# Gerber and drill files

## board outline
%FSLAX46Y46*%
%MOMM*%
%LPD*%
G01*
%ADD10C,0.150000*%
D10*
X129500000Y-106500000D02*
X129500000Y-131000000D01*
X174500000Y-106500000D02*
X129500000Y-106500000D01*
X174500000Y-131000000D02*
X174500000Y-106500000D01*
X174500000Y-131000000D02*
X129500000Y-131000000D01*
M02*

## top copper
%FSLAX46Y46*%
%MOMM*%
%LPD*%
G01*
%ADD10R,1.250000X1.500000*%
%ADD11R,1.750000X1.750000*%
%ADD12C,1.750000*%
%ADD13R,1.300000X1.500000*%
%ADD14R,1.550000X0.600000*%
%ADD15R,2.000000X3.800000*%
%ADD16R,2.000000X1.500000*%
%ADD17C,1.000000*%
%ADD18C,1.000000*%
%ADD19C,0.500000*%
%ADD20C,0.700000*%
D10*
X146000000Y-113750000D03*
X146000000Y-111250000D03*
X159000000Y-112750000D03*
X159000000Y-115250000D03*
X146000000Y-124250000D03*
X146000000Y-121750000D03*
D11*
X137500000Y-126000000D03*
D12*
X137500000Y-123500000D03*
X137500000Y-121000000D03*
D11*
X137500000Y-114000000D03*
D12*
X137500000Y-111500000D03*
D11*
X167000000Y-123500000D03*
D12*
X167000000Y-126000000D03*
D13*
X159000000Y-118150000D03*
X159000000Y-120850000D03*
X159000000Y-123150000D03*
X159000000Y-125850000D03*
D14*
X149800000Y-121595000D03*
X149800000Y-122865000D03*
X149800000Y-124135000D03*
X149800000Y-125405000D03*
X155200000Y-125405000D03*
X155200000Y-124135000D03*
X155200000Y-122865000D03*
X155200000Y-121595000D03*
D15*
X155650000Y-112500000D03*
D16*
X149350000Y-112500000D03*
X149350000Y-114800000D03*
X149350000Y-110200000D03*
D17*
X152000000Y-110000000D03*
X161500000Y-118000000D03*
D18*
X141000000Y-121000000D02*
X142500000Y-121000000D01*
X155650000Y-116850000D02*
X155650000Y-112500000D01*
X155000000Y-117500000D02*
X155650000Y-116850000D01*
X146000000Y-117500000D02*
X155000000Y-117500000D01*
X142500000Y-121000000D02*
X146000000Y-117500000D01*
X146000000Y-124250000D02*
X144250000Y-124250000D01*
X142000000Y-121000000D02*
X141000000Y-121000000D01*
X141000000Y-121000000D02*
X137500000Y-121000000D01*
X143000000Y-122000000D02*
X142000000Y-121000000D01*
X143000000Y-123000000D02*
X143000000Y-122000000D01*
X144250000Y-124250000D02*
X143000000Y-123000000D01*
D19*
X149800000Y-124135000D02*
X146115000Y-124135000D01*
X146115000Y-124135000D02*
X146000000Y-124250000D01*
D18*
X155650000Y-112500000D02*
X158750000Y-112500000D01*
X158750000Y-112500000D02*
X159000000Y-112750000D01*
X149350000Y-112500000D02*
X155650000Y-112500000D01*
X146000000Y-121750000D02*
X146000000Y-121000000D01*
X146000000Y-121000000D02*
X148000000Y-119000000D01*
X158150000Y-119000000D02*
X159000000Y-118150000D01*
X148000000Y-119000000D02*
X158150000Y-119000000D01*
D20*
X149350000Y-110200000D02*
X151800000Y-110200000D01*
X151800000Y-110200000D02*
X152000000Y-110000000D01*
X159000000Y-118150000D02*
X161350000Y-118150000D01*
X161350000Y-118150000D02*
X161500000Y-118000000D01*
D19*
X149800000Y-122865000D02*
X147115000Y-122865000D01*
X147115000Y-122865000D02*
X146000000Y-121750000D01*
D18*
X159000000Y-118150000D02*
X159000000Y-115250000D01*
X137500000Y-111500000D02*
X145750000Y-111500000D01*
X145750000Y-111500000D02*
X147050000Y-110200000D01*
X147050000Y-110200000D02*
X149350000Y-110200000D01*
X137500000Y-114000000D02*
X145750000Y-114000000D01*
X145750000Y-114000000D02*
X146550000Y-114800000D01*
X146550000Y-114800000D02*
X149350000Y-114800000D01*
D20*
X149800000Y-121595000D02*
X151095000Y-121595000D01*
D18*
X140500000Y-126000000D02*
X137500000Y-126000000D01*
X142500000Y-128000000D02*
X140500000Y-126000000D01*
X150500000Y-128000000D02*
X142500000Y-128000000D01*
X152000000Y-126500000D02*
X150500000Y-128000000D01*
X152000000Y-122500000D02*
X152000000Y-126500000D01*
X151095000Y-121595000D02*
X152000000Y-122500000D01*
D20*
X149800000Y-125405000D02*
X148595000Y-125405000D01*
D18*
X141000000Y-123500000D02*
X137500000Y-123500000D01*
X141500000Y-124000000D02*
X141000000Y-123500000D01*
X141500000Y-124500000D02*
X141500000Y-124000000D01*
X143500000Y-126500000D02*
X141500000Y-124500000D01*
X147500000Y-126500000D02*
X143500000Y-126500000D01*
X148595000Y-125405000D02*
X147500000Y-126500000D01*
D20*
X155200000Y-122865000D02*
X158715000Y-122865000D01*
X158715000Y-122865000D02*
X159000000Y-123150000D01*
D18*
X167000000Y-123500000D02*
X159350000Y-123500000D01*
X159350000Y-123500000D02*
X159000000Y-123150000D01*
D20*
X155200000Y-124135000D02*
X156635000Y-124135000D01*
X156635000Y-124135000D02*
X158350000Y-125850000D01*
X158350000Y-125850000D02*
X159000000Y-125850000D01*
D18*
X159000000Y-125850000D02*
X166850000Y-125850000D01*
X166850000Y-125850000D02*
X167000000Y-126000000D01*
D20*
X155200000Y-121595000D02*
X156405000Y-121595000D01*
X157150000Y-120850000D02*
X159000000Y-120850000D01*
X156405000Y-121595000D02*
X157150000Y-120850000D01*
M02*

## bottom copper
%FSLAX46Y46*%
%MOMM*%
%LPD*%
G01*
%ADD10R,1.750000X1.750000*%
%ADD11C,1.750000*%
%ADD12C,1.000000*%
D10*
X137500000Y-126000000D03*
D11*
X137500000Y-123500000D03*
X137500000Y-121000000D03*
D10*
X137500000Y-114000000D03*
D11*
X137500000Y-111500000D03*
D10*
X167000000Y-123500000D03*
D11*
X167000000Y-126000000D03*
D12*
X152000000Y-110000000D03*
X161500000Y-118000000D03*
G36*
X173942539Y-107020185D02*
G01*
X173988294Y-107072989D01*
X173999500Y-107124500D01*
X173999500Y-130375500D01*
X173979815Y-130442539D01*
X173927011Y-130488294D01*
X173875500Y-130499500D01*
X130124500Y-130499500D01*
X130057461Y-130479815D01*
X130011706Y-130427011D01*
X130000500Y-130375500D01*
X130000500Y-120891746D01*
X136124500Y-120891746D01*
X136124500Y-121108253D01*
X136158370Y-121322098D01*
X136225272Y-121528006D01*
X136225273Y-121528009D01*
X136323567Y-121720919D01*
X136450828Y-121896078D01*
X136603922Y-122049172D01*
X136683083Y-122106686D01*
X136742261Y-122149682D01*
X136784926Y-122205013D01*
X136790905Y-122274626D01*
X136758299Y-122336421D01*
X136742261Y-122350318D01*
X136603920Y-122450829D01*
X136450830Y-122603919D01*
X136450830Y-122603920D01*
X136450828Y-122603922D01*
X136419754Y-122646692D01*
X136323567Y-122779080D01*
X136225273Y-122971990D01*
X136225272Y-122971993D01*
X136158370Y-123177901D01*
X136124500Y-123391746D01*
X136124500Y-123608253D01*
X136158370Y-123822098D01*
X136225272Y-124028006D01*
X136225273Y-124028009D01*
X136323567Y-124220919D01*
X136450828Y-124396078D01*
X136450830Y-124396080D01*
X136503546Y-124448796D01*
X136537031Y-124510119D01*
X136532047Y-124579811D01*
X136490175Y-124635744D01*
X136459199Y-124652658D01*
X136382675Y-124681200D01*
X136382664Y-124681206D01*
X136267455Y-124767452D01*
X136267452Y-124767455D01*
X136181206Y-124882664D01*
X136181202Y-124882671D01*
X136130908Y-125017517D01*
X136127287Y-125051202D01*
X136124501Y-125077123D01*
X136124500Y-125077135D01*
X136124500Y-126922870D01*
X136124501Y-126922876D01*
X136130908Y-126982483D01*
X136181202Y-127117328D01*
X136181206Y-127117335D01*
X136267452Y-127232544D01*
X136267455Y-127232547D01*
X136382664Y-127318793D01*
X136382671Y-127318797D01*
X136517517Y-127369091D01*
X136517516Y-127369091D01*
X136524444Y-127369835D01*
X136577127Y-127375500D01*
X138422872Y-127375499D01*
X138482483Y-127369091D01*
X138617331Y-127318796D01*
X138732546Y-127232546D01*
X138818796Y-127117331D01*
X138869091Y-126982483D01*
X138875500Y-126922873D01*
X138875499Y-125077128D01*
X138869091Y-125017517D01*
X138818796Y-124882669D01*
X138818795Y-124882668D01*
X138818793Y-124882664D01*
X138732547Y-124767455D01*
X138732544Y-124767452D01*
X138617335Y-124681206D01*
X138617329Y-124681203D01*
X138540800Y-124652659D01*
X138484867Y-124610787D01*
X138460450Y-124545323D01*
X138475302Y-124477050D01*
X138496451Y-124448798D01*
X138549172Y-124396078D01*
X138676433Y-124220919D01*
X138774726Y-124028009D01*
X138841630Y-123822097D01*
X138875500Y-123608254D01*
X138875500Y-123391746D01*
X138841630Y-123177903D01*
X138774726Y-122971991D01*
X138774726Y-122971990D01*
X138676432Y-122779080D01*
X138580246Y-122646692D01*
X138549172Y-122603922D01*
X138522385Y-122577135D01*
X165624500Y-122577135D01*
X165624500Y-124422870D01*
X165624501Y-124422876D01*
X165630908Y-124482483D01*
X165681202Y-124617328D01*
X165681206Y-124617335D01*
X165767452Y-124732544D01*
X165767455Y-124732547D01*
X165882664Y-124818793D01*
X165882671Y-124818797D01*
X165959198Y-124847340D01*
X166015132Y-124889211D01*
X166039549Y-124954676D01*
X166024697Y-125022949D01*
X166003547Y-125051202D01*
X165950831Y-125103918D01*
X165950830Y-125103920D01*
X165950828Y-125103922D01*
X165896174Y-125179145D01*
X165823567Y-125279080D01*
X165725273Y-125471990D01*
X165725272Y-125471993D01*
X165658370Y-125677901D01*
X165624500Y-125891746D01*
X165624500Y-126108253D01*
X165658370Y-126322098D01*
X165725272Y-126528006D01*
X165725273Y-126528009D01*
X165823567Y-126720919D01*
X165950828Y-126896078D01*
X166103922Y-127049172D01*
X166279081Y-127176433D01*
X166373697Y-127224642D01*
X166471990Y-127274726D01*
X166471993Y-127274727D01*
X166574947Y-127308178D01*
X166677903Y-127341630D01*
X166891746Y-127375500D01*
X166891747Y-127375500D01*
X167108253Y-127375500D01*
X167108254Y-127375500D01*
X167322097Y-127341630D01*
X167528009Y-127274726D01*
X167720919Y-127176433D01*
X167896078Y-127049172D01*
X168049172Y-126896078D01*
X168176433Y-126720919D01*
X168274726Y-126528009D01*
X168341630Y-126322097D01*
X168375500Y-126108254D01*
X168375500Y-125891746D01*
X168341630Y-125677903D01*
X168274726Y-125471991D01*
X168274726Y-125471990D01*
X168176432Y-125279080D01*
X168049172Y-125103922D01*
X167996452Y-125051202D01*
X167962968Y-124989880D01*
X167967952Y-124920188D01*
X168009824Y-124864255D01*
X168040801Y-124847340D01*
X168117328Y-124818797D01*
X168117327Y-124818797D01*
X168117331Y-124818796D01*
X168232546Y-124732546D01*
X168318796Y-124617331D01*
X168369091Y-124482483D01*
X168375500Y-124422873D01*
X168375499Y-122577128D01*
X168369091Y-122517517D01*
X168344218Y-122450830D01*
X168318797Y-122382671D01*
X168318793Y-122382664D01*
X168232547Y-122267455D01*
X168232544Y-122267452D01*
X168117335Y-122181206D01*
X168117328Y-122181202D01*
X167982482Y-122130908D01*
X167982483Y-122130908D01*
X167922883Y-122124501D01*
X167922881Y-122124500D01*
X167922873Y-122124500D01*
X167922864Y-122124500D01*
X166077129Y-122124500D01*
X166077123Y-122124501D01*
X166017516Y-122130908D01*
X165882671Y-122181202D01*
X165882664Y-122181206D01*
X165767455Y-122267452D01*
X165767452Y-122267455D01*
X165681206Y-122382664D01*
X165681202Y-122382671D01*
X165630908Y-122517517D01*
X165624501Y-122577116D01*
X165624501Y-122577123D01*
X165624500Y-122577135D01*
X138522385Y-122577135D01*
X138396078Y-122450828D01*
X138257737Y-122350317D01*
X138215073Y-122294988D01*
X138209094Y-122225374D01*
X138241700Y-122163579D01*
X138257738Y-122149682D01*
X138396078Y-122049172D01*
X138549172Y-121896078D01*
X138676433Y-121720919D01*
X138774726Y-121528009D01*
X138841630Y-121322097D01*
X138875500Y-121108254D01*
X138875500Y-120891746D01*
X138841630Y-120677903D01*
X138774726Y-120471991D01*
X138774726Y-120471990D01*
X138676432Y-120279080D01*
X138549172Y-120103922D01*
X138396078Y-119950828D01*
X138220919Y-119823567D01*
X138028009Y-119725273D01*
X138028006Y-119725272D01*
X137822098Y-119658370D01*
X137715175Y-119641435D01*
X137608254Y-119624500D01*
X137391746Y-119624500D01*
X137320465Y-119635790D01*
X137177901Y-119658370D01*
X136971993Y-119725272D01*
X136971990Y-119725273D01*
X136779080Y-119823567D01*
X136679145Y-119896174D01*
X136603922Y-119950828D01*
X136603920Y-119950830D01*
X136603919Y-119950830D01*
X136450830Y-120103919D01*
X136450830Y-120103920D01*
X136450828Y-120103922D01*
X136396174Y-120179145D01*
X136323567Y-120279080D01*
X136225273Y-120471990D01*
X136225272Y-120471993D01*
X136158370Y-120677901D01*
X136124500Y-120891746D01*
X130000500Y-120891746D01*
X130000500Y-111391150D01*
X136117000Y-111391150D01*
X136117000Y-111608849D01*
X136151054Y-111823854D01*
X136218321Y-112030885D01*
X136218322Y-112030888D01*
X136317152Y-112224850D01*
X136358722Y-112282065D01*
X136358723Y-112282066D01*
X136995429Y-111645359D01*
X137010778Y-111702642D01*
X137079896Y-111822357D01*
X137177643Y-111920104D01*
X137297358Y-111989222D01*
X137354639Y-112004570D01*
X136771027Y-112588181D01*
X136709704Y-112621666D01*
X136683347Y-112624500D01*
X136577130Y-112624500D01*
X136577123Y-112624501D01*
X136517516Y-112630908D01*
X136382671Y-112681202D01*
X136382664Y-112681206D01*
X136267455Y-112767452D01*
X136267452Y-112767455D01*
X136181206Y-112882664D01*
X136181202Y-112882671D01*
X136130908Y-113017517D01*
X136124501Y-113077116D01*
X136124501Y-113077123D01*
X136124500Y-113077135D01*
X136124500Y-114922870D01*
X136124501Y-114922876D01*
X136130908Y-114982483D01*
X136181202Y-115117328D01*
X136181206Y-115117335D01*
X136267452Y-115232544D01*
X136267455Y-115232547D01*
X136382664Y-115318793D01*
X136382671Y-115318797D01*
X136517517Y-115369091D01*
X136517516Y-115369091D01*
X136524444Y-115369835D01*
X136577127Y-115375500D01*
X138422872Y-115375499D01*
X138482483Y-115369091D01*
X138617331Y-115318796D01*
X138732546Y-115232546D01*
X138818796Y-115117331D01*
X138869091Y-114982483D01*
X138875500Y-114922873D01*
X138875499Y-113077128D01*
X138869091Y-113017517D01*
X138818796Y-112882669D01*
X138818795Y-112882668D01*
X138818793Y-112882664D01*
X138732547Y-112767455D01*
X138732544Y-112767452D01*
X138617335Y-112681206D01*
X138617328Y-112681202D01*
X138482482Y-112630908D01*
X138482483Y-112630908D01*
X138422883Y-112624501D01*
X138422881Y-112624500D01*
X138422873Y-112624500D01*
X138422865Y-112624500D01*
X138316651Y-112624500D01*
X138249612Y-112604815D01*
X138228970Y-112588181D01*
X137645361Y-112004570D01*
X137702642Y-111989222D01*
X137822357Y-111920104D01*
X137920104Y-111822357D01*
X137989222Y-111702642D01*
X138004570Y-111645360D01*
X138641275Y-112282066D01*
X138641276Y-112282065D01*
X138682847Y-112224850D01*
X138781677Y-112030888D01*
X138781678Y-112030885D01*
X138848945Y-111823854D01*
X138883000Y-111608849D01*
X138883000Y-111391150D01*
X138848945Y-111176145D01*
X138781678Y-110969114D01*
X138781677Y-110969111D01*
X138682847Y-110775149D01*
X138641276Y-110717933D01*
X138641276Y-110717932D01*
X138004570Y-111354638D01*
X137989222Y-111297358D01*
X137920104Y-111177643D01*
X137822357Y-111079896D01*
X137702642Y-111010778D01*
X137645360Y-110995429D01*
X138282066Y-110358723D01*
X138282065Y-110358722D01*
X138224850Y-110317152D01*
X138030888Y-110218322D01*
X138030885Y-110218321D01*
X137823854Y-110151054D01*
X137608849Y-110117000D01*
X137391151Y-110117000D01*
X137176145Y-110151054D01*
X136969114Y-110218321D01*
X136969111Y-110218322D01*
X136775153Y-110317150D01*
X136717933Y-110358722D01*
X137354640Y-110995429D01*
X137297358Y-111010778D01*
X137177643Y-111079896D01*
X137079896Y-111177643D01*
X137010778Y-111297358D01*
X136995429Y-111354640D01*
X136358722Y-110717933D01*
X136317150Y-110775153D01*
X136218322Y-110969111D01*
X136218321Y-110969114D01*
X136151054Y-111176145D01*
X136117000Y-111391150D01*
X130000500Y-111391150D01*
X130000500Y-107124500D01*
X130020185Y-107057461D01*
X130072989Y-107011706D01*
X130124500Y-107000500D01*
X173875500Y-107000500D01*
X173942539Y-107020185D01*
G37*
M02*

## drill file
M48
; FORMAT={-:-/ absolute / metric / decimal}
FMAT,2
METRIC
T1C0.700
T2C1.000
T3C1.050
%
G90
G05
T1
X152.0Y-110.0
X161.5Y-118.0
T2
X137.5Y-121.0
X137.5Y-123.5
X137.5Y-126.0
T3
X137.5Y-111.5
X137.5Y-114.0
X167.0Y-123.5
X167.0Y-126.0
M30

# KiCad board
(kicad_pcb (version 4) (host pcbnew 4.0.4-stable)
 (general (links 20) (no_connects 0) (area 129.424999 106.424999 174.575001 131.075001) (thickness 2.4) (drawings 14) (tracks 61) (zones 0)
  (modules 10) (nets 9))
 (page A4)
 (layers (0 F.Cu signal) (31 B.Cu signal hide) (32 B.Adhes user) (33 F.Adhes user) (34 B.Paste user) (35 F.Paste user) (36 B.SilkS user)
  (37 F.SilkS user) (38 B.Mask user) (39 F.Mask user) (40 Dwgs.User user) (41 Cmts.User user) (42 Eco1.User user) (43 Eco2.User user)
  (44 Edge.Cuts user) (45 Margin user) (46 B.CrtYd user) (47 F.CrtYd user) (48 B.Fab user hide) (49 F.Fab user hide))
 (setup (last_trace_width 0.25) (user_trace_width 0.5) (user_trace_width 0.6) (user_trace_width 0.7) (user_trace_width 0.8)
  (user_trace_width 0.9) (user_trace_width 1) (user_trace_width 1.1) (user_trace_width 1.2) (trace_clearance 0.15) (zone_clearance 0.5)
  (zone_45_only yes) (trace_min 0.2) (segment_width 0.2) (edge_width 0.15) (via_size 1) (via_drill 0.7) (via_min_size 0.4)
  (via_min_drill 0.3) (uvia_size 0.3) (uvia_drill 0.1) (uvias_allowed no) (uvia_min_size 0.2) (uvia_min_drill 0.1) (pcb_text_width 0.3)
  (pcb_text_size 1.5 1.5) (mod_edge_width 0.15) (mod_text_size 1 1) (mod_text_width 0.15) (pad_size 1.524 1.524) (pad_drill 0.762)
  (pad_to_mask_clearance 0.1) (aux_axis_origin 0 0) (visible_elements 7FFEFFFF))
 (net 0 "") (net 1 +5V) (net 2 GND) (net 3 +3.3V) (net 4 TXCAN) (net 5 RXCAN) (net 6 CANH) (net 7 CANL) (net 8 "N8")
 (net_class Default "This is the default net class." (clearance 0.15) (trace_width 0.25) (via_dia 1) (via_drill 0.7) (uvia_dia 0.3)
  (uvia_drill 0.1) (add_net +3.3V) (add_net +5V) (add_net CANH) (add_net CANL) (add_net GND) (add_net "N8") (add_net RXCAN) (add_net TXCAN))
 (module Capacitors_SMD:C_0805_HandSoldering (layer F.Cu) (at 146 112.5 90)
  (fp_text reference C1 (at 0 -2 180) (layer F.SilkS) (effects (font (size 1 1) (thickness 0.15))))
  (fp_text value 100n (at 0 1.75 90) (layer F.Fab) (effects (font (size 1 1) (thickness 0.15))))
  (pad 1 smd rect (at -1.25 0 90) (size 1.5 1.25) (layers F.Cu F.Paste F.Mask) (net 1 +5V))
  (pad 2 smd rect (at 1.25 0 90) (size 1.5 1.25) (layers F.Cu F.Paste F.Mask) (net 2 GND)))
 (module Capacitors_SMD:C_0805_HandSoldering (layer F.Cu) (at 159 114 270)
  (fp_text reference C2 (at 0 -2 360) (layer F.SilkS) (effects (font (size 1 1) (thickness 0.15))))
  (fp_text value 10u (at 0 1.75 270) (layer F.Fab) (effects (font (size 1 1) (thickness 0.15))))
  (pad 1 smd rect (at -1.25 0 270) (size 1.5 1.25) (layers F.Cu F.Paste F.Mask) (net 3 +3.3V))
  (pad 2 smd rect (at 1.25 0 270) (size 1.5 1.25) (layers F.Cu F.Paste F.Mask) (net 2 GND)))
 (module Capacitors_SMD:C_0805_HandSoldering (layer F.Cu) (at 146 123 90)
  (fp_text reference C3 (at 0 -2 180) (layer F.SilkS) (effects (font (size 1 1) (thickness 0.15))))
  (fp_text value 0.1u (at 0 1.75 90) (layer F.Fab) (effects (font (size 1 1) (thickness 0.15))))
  (pad 1 smd rect (at -1.25 0 90) (size 1.5 1.25) (layers F.Cu F.Paste F.Mask) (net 3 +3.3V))
  (pad 2 smd rect (at 1.25 0 90) (size 1.5 1.25) (layers F.Cu F.Paste F.Mask) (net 2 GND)))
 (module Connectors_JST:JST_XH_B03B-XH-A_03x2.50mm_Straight (layer F.Cu) (at 137.5 126 90)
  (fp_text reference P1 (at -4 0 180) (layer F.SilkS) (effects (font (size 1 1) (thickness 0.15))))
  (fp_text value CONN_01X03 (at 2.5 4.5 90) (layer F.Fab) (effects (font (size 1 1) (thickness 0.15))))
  (pad 1 thru_hole rect (at 0 0 90) (size 1.75 1.75) (drill 1) (layers *.Cu *.Mask) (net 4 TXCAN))
  (pad 2 thru_hole circle (at 2.5 0 90) (size 1.75 1.75) (drill 1) (layers *.Cu *.Mask) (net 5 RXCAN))
  (pad 3 thru_hole circle (at 5 0 90) (size 1.75 1.75) (drill 1) (layers *.Cu *.Mask) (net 3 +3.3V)))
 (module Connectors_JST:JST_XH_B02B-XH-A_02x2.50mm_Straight (layer F.Cu) (at 137.5 114 90)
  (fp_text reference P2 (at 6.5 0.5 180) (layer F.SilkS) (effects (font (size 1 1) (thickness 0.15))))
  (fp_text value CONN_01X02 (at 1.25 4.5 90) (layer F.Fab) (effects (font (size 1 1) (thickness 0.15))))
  (pad 1 thru_hole rect (at 0 0 90) (size 1.75 1.75) (drill 1.05) (layers *.Cu *.Mask) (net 1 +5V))
  (pad 2 thru_hole circle (at 2.5 0 90) (size 1.75 1.75) (drill 1.05) (layers *.Cu *.Mask) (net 2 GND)))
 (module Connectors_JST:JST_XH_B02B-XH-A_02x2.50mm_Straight (layer F.Cu) (at 167 123.5 270)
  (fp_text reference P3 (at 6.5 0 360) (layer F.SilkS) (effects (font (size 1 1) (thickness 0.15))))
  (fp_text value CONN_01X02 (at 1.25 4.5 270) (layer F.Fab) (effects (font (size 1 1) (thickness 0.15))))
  (pad 1 thru_hole rect (at 0 0 270) (size 1.75 1.75) (drill 1.05) (layers *.Cu *.Mask) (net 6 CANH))
  (pad 2 thru_hole circle (at 2.5 0 270) (size 1.75 1.75) (drill 1.05) (layers *.Cu *.Mask) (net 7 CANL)))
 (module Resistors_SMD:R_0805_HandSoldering (layer F.Cu) (at 159 119.5 270)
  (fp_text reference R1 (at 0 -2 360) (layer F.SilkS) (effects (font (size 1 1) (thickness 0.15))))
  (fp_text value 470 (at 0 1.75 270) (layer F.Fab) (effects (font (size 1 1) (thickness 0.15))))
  (pad 1 smd rect (at -1.35 0 270) (size 1.5 1.3) (layers F.Cu F.Paste F.Mask) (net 2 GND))
  (pad 2 smd rect (at 1.35 0 270) (size 1.5 1.3) (layers F.Cu F.Paste F.Mask) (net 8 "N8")))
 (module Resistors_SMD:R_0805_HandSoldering (layer F.Cu) (at 159 124.5 270)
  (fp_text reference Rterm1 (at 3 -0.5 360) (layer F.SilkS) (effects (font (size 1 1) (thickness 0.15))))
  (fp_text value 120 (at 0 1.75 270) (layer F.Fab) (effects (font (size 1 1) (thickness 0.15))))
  (pad 1 smd rect (at -1.35 0 270) (size 1.5 1.3) (layers F.Cu F.Paste F.Mask) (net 6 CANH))
  (pad 2 smd rect (at 1.35 0 270) (size 1.5 1.3) (layers F.Cu F.Paste F.Mask) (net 7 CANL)))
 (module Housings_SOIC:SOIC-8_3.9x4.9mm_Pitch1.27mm (layer F.Cu) (at 152.5 123.5)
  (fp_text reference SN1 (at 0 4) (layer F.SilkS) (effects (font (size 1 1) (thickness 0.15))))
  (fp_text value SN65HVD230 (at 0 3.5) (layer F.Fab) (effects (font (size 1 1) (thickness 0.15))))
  (pad 1 smd rect (at -2.7 -1.905) (size 1.55 0.6) (layers F.Cu F.Paste F.Mask) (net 4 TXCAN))
  (pad 2 smd rect (at -2.7 -0.635) (size 1.55 0.6) (layers F.Cu F.Paste F.Mask) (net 2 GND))
  (pad 3 smd rect (at -2.7 0.635) (size 1.55 0.6) (layers F.Cu F.Paste F.Mask) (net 3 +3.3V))
  (pad 4 smd rect (at -2.7 1.905) (size 1.55 0.6) (layers F.Cu F.Paste F.Mask) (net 5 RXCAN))
  (pad 5 smd rect (at 2.7 1.905) (size 1.55 0.6) (layers F.Cu F.Paste F.Mask))
  (pad 6 smd rect (at 2.7 0.635) (size 1.55 0.6) (layers F.Cu F.Paste F.Mask) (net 7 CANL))
  (pad 7 smd rect (at 2.7 -0.635) (size 1.55 0.6) (layers F.Cu F.Paste F.Mask) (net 6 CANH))
  (pad 8 smd rect (at 2.7 -1.905) (size 1.55 0.6) (layers F.Cu F.Paste F.Mask) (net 8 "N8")))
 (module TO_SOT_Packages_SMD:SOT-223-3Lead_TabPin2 (layer F.Cu) (at 152.5 112.5)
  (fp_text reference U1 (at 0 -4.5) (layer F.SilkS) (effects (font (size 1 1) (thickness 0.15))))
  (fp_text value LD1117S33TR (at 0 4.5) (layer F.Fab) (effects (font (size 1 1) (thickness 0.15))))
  (pad 2 smd rect (at 3.15 0) (size 2 3.8) (layers F.Cu F.Paste F.Mask) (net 3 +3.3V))
  (pad 2 smd rect (at -3.15 0) (size 2 1.5) (layers F.Cu F.Paste F.Mask) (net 3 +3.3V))
  (pad 3 smd rect (at -3.15 2.3) (size 2 1.5) (layers F.Cu F.Paste F.Mask) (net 1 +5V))
  (pad 1 smd rect (at -3.15 -2.3) (size 2 1.5) (layers F.Cu F.Paste F.Mask) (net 2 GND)))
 (gr_line (start 129.5 106.5) (end 129.5 131) (angle 90) (layer Edge.Cuts) (width 0.15))
 (gr_line (start 174.5 106.5) (end 129.5 106.5) (angle 90) (layer Edge.Cuts) (width 0.15))
 (gr_line (start 174.5 131) (end 174.5 106.5) (angle 90) (layer Edge.Cuts) (width 0.15))
 (gr_line (start 174.5 131) (end 129.5 131) (angle 90) (layer Edge.Cuts) (width 0.15))
 (segment (start 141 121) (end 142.5 121) (width 1) (layer F.Cu) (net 3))
 (segment (start 155.65 116.85) (end 155.65 112.5) (width 1) (layer F.Cu) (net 3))
 (segment (start 155 117.5) (end 155.65 116.85) (width 1) (layer F.Cu) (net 3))
 (segment (start 146 117.5) (end 155 117.5) (width 1) (layer F.Cu) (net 3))
 (segment (start 142.5 121) (end 146 117.5) (width 1) (layer F.Cu) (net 3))
 (segment (start 146 124.25) (end 144.25 124.25) (width 1) (layer F.Cu) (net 3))
 (segment (start 142 121) (end 141 121) (width 1) (layer F.Cu) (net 3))
 (segment (start 141 121) (end 137.5 121) (width 1) (layer F.Cu) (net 3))
 (segment (start 143 122) (end 142 121) (width 1) (layer F.Cu) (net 3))
 (segment (start 143 123) (end 143 122) (width 1) (layer F.Cu) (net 3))
 (segment (start 144.25 124.25) (end 143 123) (width 1) (layer F.Cu) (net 3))
 (segment (start 149.8 124.135) (end 146.115 124.135) (width 0.5) (layer F.Cu) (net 3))
 (segment (start 146.115 124.135) (end 146 124.25) (width 0.5) (layer F.Cu) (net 3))
 (segment (start 155.65 112.5) (end 158.75 112.5) (width 1) (layer F.Cu) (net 3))
 (segment (start 158.75 112.5) (end 159 112.75) (width 1) (layer F.Cu) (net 3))
 (segment (start 149.35 112.5) (end 155.65 112.5) (width 1) (layer F.Cu) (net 3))
 (segment (start 146 121.75) (end 146 121) (width 1) (layer F.Cu) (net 2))
 (segment (start 146 121) (end 148 119) (width 1) (layer F.Cu) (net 2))
 (segment (start 158.15 119) (end 159 118.15) (width 1) (layer F.Cu) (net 2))
 (segment (start 148 119) (end 158.15 119) (width 1) (layer F.Cu) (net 2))
 (segment (start 149.35 110.2) (end 151.8 110.2) (width 0.7) (layer F.Cu) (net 2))
 (via (at 152 110) (size 1) (drill 0.7) (layers F.Cu B.Cu) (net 2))
 (segment (start 151.8 110.2) (end 152 110) (width 0.7) (layer F.Cu) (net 2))
 (segment (start 159 118.15) (end 161.35 118.15) (width 0.7) (layer F.Cu) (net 2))
 (via (at 161.5 118) (size 1) (drill 0.7) (layers F.Cu B.Cu) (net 2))
 (segment (start 161.35 118.15) (end 161.5 118) (width 0.7) (layer F.Cu) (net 2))
 (segment (start 149.8 122.865) (end 147.115 122.865) (width 0.5) (layer F.Cu) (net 2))
 (segment (start 147.115 122.865) (end 146 121.75) (width 0.5) (layer F.Cu) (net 2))
 (segment (start 159 118.15) (end 159 115.25) (width 1) (layer F.Cu) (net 2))
 (segment (start 137.5 111.5) (end 145.75 111.5) (width 1) (layer F.Cu) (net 2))
 (segment (start 145.75 111.5) (end 147.05 110.2) (width 1) (layer F.Cu) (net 2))
 (segment (start 147.05 110.2) (end 149.35 110.2) (width 1) (layer F.Cu) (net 2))
 (segment (start 137.5 114) (end 145.75 114) (width 1) (layer F.Cu) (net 1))
 (segment (start 145.75 114) (end 146.55 114.8) (width 1) (layer F.Cu) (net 1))
 (segment (start 146.55 114.8) (end 149.35 114.8) (width 1) (layer F.Cu) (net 1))
 (segment (start 149.8 121.595) (end 151.095 121.595) (width 0.7) (layer F.Cu) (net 4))
 (segment (start 140.5 126) (end 137.5 126) (width 1) (layer F.Cu) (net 4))
 (segment (start 142.5 128) (end 140.5 126) (width 1) (layer F.Cu) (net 4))
 (segment (start 150.5 128) (end 142.5 128) (width 1) (layer F.Cu) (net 4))
 (segment (start 152 126.5) (end 150.5 128) (width 1) (layer F.Cu) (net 4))
 (segment (start 152 122.5) (end 152 126.5) (width 1) (layer F.Cu) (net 4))
 (segment (start 151.095 121.595) (end 152 122.5) (width 1) (layer F.Cu) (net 4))
 (segment (start 149.8 125.405) (end 148.595 125.405) (width 0.7) (layer F.Cu) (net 5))
 (segment (start 141 123.5) (end 137.5 123.5) (width 1) (layer F.Cu) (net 5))
 (segment (start 141.5 124) (end 141 123.5) (width 1) (layer F.Cu) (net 5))
 (segment (start 141.5 124.5) (end 141.5 124) (width 1) (layer F.Cu) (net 5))
 (segment (start 143.5 126.5) (end 141.5 124.5) (width 1) (layer F.Cu) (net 5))
 (segment (start 147.5 126.5) (end 143.5 126.5) (width 1) (layer F.Cu) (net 5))
 (segment (start 148.595 125.405) (end 147.5 126.5) (width 1) (layer F.Cu) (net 5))
 (segment (start 155.2 122.865) (end 158.715 122.865) (width 0.7) (layer F.Cu) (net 6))
 (segment (start 158.715 122.865) (end 159 123.15) (width 0.7) (layer F.Cu) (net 6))
 (segment (start 167 123.5) (end 159.35 123.5) (width 1) (layer F.Cu) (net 6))
 (segment (start 159.35 123.5) (end 159 123.15) (width 1) (layer F.Cu) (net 6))
 (segment (start 155.2 124.135) (end 156.635 124.135) (width 0.7) (layer F.Cu) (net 7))
 (segment (start 156.635 124.135) (end 158.35 125.85) (width 0.7) (layer F.Cu) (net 7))
 (segment (start 158.35 125.85) (end 159 125.85) (width 0.7) (layer F.Cu) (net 7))
 (segment (start 159 125.85) (end 166.85 125.85) (width 1) (layer F.Cu) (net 7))
 (segment (start 166.85 125.85) (end 167 126) (width 1) (layer F.Cu) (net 7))
 (segment (start 155.2 121.595) (end 156.405 121.595) (width 0.7) (layer F.Cu) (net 8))
 (segment (start 157.15 120.85) (end 159 120.85) (width 0.7) (layer F.Cu) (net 8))
 (segment (start 156.405 121.595) (end 157.15 120.85) (width 0.7) (layer F.Cu) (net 8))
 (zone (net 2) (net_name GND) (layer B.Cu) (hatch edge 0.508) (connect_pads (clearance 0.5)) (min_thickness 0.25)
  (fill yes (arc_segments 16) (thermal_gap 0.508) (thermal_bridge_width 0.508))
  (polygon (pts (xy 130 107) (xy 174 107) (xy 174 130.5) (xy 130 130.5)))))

